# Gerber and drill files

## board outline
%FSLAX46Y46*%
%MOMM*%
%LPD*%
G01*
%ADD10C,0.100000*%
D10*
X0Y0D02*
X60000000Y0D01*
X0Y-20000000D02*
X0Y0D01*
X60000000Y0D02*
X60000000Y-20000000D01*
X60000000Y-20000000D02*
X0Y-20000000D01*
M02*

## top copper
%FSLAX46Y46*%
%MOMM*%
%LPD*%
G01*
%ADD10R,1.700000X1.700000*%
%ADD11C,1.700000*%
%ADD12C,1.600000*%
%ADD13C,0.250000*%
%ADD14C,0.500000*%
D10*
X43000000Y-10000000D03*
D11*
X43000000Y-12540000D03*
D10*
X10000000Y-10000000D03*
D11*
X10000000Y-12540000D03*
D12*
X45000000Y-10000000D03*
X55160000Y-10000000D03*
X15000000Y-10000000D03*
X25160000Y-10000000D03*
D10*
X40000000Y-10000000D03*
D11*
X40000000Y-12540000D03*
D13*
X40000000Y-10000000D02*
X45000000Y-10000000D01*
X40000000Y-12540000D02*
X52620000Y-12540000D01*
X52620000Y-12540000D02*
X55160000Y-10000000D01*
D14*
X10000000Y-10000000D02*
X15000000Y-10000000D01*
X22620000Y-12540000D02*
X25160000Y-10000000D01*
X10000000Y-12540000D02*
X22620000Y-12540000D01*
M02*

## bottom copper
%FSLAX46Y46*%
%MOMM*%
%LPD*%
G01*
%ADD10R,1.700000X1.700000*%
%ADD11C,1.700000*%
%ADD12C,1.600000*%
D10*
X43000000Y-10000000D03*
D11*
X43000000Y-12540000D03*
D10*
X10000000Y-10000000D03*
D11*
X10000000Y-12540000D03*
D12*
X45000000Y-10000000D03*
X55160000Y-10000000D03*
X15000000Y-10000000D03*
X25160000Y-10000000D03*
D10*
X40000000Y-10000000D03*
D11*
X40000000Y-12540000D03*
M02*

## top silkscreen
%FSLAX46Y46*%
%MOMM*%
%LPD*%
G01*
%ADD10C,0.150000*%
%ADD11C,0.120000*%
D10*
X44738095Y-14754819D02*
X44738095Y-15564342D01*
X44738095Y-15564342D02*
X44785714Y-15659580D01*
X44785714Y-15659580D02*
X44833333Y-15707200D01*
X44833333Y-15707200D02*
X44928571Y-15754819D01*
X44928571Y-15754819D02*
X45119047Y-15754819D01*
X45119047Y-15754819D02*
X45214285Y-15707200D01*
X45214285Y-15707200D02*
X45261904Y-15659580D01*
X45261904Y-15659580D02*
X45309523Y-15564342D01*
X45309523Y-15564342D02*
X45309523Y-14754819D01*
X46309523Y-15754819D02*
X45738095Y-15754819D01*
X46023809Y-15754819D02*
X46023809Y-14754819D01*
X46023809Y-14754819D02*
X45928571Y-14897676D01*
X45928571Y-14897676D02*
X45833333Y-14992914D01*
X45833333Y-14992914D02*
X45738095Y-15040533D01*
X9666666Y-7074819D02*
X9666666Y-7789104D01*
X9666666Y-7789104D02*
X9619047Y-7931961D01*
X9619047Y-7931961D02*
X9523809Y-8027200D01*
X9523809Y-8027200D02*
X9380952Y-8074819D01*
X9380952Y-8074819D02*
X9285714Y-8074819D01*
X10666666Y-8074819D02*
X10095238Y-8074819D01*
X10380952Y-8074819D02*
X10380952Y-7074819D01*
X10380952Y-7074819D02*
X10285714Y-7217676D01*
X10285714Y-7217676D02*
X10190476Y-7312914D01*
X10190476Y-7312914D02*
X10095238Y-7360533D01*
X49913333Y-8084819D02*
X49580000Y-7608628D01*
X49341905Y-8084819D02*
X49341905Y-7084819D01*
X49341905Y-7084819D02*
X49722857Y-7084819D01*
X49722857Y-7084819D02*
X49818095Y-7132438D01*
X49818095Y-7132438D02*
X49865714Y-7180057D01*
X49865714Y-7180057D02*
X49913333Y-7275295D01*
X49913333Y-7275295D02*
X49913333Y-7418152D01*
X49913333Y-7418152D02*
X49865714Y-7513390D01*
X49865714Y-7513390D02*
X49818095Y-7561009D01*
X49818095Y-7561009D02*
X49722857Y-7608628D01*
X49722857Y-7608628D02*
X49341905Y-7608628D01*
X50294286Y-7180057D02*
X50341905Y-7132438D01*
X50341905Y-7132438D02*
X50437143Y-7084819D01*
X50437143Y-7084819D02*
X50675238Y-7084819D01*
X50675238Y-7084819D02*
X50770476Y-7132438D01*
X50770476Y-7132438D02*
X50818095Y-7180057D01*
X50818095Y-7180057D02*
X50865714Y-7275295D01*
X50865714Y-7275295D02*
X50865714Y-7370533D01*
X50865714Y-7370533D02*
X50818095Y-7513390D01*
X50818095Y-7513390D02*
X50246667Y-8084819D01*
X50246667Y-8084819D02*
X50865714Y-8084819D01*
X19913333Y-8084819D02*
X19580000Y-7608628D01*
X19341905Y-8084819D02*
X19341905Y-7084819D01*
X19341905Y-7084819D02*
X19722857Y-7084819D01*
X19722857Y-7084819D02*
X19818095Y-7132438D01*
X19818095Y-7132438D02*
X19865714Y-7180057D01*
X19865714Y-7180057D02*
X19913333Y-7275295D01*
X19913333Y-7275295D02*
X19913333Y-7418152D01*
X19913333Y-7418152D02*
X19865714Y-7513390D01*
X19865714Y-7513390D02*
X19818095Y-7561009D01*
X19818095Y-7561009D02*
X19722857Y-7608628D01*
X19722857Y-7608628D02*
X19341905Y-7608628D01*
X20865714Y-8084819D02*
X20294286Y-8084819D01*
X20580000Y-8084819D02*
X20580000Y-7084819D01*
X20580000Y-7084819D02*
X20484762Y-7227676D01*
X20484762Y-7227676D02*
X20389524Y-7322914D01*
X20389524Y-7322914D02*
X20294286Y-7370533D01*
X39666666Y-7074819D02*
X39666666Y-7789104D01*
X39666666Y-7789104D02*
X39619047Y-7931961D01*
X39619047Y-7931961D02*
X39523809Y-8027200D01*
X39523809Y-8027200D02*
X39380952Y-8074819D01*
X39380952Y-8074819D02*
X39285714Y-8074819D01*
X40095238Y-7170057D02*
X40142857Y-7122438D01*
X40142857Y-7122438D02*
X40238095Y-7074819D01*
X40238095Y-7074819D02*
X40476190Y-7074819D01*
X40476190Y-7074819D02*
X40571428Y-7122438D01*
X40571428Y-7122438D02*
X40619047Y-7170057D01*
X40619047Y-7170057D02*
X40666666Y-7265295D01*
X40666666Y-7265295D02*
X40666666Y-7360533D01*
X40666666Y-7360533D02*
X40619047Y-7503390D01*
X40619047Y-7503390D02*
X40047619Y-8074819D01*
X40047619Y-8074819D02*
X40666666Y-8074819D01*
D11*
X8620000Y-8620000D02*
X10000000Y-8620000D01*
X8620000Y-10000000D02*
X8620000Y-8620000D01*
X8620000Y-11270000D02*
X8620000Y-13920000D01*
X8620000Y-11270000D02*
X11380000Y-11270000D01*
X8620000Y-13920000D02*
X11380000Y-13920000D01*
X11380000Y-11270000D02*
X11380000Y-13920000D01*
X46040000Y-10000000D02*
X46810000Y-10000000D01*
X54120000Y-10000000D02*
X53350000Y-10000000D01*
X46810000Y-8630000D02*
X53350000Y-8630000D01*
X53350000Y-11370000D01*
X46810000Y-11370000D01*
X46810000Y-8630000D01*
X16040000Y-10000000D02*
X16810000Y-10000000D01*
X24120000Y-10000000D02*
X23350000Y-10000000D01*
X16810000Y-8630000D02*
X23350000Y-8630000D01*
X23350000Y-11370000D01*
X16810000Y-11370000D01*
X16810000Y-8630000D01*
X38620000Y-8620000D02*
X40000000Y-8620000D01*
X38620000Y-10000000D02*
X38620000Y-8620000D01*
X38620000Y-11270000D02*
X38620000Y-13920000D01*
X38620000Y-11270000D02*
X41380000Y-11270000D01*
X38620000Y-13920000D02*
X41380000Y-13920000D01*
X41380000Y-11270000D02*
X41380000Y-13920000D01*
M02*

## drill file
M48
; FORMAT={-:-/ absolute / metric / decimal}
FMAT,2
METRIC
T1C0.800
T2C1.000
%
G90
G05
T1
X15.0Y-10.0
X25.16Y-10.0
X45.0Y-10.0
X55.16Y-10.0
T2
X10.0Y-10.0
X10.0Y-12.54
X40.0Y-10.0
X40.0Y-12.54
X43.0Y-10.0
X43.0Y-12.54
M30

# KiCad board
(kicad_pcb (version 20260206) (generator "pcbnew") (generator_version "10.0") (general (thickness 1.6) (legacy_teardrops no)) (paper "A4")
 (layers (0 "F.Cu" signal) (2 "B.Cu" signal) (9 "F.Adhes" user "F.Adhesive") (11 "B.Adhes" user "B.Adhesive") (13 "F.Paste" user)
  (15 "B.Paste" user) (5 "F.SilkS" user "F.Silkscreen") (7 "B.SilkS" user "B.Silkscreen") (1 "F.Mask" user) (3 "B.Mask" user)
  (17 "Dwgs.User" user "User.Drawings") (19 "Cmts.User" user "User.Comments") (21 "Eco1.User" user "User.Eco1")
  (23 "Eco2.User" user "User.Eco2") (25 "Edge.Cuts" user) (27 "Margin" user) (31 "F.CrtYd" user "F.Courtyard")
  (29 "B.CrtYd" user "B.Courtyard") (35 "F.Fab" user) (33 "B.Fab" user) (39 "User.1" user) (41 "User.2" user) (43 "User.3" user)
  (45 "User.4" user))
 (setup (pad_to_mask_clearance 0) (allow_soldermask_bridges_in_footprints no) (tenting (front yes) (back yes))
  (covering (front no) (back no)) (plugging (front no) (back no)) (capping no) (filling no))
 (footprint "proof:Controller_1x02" (layer "F.Cu") (at 43 10)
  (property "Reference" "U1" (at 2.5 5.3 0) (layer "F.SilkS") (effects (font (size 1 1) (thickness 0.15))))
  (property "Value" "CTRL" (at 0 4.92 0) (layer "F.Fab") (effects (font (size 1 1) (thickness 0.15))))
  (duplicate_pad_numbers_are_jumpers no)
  (pad "1" thru_hole rect (at 0 0) (size 1.7 1.7) (drill 1) (layers "*.Cu" "*.Mask") (remove_unused_layers no) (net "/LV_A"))
  (pad "2" thru_hole circle (at 0 2.54) (size 1.7 1.7) (drill 1) (layers "*.Cu" "*.Mask") (remove_unused_layers no) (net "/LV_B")))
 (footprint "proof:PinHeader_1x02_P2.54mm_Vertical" (layer "F.Cu") (at 10 10)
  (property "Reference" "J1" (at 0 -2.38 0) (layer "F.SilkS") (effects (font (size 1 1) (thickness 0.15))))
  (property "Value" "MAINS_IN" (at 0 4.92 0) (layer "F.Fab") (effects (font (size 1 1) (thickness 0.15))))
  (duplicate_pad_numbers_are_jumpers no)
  (fp_line (start -1.38 -1.38) (end 0 -1.38) (stroke (width 0.12) (type solid)) (layer "F.SilkS"))
  (fp_line (start -1.38 0) (end -1.38 -1.38) (stroke (width 0.12) (type solid)) (layer "F.SilkS"))
  (fp_line (start -1.38 1.27) (end -1.38 3.92) (stroke (width 0.12) (type solid)) (layer "F.SilkS"))
  (fp_line (start -1.38 1.27) (end 1.38 1.27) (stroke (width 0.12) (type solid)) (layer "F.SilkS"))
  (fp_line (start -1.38 3.92) (end 1.38 3.92) (stroke (width 0.12) (type solid)) (layer "F.SilkS"))
  (fp_line (start 1.38 1.27) (end 1.38 3.92) (stroke (width 0.12) (type solid)) (layer "F.SilkS"))
  (pad "1" thru_hole rect (at 0 0) (size 1.7 1.7) (drill 1) (layers "*.Cu" "*.Mask") (remove_unused_layers no) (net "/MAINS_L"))
  (pad "2" thru_hole circle (at 0 2.54) (size 1.7 1.7) (drill 1) (layers "*.Cu" "*.Mask") (remove_unused_layers no) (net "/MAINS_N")))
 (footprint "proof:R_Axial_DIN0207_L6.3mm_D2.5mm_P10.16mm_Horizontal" (layer "F.Cu") (at 45 10)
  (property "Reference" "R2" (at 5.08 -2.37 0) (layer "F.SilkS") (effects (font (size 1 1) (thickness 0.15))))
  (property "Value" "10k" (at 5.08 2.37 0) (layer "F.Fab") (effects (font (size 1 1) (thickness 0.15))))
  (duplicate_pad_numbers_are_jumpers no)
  (fp_line (start 1.04 0) (end 1.81 0) (stroke (width 0.12) (type solid)) (layer "F.SilkS"))
  (fp_line (start 9.12 0) (end 8.35 0) (stroke (width 0.12) (type solid)) (layer "F.SilkS"))
  (fp_rect (start 1.81 -1.37) (end 8.35 1.37) (stroke (width 0.12) (type solid)) (fill no) (layer "F.SilkS"))
  (pad "1" thru_hole circle (at 0 0) (size 1.6 1.6) (drill 0.8) (layers "*.Cu" "*.Mask") (remove_unused_layers no) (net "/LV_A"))
  (pad "2" thru_hole circle (at 10.16 0) (size 1.6 1.6) (drill 0.8) (layers "*.Cu" "*.Mask") (remove_unused_layers no) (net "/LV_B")))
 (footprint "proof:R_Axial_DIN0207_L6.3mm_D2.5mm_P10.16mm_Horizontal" (layer "F.Cu") (at 15 10)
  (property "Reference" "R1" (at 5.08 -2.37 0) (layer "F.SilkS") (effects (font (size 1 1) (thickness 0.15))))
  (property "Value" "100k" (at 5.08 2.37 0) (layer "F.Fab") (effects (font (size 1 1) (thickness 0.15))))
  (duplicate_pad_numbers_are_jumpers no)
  (fp_line (start 1.04 0) (end 1.81 0) (stroke (width 0.12) (type solid)) (layer "F.SilkS"))
  (fp_line (start 9.12 0) (end 8.35 0) (stroke (width 0.12) (type solid)) (layer "F.SilkS"))
  (fp_rect (start 1.81 -1.37) (end 8.35 1.37) (stroke (width 0.12) (type solid)) (fill no) (layer "F.SilkS"))
  (pad "1" thru_hole circle (at 0 0) (size 1.6 1.6) (drill 0.8) (layers "*.Cu" "*.Mask") (remove_unused_layers no) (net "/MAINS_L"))
  (pad "2" thru_hole circle (at 10.16 0) (size 1.6 1.6) (drill 0.8) (layers "*.Cu" "*.Mask") (remove_unused_layers no) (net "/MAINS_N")))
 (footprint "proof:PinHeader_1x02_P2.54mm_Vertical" (layer "F.Cu") (at 40 10)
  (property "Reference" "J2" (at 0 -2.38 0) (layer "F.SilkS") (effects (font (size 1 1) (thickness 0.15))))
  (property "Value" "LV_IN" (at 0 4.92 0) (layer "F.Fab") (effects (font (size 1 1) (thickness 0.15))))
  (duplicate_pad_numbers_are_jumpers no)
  (fp_line (start -1.38 -1.38) (end 0 -1.38) (stroke (width 0.12) (type solid)) (layer "F.SilkS"))
  (fp_line (start -1.38 0) (end -1.38 -1.38) (stroke (width 0.12) (type solid)) (layer "F.SilkS"))
  (fp_line (start -1.38 1.27) (end -1.38 3.92) (stroke (width 0.12) (type solid)) (layer "F.SilkS"))
  (fp_line (start -1.38 1.27) (end 1.38 1.27) (stroke (width 0.12) (type solid)) (layer "F.SilkS"))
  (fp_line (start -1.38 3.92) (end 1.38 3.92) (stroke (width 0.12) (type solid)) (layer "F.SilkS"))
  (fp_line (start 1.38 1.27) (end 1.38 3.92) (stroke (width 0.12) (type solid)) (layer "F.SilkS"))
  (pad "1" thru_hole rect (at 0 0) (size 1.7 1.7) (drill 1) (layers "*.Cu" "*.Mask") (remove_unused_layers no) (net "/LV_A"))
  (pad "2" thru_hole circle (at 0 2.54) (size 1.7 1.7) (drill 1) (layers "*.Cu" "*.Mask") (remove_unused_layers no) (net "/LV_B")))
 (gr_line (start 0 0) (end 60 0) (stroke (width 0.1) (type default)) (layer "Edge.Cuts"))
 (gr_line (start 0 20) (end 0 0) (stroke (width 0.1) (type default)) (layer "Edge.Cuts"))
 (gr_line (start 60 0) (end 60 20) (stroke (width 0.1) (type default)) (layer "Edge.Cuts"))
 (gr_line (start 60 20) (end 0 20) (stroke (width 0.1) (type default)) (layer "Edge.Cuts"))
 (segment (start 40 10) (end 45 10) (width 0.25) (layer "F.Cu") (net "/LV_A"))
 (segment (start 40 12.54) (end 52.62 12.54) (width 0.25) (layer "F.Cu") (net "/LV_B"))
 (segment (start 52.62 12.54) (end 55.16 10) (width 0.25) (layer "F.Cu") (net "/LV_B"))
 (segment (start 10 10) (end 15 10) (width 0.5) (layer "F.Cu") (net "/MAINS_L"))
 (segment (start 22.62 12.54) (end 25.16 10) (width 0.5) (layer "F.Cu") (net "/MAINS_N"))
 (segment (start 10 12.54) (end 22.62 12.54) (width 0.5) (layer "F.Cu") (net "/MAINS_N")))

